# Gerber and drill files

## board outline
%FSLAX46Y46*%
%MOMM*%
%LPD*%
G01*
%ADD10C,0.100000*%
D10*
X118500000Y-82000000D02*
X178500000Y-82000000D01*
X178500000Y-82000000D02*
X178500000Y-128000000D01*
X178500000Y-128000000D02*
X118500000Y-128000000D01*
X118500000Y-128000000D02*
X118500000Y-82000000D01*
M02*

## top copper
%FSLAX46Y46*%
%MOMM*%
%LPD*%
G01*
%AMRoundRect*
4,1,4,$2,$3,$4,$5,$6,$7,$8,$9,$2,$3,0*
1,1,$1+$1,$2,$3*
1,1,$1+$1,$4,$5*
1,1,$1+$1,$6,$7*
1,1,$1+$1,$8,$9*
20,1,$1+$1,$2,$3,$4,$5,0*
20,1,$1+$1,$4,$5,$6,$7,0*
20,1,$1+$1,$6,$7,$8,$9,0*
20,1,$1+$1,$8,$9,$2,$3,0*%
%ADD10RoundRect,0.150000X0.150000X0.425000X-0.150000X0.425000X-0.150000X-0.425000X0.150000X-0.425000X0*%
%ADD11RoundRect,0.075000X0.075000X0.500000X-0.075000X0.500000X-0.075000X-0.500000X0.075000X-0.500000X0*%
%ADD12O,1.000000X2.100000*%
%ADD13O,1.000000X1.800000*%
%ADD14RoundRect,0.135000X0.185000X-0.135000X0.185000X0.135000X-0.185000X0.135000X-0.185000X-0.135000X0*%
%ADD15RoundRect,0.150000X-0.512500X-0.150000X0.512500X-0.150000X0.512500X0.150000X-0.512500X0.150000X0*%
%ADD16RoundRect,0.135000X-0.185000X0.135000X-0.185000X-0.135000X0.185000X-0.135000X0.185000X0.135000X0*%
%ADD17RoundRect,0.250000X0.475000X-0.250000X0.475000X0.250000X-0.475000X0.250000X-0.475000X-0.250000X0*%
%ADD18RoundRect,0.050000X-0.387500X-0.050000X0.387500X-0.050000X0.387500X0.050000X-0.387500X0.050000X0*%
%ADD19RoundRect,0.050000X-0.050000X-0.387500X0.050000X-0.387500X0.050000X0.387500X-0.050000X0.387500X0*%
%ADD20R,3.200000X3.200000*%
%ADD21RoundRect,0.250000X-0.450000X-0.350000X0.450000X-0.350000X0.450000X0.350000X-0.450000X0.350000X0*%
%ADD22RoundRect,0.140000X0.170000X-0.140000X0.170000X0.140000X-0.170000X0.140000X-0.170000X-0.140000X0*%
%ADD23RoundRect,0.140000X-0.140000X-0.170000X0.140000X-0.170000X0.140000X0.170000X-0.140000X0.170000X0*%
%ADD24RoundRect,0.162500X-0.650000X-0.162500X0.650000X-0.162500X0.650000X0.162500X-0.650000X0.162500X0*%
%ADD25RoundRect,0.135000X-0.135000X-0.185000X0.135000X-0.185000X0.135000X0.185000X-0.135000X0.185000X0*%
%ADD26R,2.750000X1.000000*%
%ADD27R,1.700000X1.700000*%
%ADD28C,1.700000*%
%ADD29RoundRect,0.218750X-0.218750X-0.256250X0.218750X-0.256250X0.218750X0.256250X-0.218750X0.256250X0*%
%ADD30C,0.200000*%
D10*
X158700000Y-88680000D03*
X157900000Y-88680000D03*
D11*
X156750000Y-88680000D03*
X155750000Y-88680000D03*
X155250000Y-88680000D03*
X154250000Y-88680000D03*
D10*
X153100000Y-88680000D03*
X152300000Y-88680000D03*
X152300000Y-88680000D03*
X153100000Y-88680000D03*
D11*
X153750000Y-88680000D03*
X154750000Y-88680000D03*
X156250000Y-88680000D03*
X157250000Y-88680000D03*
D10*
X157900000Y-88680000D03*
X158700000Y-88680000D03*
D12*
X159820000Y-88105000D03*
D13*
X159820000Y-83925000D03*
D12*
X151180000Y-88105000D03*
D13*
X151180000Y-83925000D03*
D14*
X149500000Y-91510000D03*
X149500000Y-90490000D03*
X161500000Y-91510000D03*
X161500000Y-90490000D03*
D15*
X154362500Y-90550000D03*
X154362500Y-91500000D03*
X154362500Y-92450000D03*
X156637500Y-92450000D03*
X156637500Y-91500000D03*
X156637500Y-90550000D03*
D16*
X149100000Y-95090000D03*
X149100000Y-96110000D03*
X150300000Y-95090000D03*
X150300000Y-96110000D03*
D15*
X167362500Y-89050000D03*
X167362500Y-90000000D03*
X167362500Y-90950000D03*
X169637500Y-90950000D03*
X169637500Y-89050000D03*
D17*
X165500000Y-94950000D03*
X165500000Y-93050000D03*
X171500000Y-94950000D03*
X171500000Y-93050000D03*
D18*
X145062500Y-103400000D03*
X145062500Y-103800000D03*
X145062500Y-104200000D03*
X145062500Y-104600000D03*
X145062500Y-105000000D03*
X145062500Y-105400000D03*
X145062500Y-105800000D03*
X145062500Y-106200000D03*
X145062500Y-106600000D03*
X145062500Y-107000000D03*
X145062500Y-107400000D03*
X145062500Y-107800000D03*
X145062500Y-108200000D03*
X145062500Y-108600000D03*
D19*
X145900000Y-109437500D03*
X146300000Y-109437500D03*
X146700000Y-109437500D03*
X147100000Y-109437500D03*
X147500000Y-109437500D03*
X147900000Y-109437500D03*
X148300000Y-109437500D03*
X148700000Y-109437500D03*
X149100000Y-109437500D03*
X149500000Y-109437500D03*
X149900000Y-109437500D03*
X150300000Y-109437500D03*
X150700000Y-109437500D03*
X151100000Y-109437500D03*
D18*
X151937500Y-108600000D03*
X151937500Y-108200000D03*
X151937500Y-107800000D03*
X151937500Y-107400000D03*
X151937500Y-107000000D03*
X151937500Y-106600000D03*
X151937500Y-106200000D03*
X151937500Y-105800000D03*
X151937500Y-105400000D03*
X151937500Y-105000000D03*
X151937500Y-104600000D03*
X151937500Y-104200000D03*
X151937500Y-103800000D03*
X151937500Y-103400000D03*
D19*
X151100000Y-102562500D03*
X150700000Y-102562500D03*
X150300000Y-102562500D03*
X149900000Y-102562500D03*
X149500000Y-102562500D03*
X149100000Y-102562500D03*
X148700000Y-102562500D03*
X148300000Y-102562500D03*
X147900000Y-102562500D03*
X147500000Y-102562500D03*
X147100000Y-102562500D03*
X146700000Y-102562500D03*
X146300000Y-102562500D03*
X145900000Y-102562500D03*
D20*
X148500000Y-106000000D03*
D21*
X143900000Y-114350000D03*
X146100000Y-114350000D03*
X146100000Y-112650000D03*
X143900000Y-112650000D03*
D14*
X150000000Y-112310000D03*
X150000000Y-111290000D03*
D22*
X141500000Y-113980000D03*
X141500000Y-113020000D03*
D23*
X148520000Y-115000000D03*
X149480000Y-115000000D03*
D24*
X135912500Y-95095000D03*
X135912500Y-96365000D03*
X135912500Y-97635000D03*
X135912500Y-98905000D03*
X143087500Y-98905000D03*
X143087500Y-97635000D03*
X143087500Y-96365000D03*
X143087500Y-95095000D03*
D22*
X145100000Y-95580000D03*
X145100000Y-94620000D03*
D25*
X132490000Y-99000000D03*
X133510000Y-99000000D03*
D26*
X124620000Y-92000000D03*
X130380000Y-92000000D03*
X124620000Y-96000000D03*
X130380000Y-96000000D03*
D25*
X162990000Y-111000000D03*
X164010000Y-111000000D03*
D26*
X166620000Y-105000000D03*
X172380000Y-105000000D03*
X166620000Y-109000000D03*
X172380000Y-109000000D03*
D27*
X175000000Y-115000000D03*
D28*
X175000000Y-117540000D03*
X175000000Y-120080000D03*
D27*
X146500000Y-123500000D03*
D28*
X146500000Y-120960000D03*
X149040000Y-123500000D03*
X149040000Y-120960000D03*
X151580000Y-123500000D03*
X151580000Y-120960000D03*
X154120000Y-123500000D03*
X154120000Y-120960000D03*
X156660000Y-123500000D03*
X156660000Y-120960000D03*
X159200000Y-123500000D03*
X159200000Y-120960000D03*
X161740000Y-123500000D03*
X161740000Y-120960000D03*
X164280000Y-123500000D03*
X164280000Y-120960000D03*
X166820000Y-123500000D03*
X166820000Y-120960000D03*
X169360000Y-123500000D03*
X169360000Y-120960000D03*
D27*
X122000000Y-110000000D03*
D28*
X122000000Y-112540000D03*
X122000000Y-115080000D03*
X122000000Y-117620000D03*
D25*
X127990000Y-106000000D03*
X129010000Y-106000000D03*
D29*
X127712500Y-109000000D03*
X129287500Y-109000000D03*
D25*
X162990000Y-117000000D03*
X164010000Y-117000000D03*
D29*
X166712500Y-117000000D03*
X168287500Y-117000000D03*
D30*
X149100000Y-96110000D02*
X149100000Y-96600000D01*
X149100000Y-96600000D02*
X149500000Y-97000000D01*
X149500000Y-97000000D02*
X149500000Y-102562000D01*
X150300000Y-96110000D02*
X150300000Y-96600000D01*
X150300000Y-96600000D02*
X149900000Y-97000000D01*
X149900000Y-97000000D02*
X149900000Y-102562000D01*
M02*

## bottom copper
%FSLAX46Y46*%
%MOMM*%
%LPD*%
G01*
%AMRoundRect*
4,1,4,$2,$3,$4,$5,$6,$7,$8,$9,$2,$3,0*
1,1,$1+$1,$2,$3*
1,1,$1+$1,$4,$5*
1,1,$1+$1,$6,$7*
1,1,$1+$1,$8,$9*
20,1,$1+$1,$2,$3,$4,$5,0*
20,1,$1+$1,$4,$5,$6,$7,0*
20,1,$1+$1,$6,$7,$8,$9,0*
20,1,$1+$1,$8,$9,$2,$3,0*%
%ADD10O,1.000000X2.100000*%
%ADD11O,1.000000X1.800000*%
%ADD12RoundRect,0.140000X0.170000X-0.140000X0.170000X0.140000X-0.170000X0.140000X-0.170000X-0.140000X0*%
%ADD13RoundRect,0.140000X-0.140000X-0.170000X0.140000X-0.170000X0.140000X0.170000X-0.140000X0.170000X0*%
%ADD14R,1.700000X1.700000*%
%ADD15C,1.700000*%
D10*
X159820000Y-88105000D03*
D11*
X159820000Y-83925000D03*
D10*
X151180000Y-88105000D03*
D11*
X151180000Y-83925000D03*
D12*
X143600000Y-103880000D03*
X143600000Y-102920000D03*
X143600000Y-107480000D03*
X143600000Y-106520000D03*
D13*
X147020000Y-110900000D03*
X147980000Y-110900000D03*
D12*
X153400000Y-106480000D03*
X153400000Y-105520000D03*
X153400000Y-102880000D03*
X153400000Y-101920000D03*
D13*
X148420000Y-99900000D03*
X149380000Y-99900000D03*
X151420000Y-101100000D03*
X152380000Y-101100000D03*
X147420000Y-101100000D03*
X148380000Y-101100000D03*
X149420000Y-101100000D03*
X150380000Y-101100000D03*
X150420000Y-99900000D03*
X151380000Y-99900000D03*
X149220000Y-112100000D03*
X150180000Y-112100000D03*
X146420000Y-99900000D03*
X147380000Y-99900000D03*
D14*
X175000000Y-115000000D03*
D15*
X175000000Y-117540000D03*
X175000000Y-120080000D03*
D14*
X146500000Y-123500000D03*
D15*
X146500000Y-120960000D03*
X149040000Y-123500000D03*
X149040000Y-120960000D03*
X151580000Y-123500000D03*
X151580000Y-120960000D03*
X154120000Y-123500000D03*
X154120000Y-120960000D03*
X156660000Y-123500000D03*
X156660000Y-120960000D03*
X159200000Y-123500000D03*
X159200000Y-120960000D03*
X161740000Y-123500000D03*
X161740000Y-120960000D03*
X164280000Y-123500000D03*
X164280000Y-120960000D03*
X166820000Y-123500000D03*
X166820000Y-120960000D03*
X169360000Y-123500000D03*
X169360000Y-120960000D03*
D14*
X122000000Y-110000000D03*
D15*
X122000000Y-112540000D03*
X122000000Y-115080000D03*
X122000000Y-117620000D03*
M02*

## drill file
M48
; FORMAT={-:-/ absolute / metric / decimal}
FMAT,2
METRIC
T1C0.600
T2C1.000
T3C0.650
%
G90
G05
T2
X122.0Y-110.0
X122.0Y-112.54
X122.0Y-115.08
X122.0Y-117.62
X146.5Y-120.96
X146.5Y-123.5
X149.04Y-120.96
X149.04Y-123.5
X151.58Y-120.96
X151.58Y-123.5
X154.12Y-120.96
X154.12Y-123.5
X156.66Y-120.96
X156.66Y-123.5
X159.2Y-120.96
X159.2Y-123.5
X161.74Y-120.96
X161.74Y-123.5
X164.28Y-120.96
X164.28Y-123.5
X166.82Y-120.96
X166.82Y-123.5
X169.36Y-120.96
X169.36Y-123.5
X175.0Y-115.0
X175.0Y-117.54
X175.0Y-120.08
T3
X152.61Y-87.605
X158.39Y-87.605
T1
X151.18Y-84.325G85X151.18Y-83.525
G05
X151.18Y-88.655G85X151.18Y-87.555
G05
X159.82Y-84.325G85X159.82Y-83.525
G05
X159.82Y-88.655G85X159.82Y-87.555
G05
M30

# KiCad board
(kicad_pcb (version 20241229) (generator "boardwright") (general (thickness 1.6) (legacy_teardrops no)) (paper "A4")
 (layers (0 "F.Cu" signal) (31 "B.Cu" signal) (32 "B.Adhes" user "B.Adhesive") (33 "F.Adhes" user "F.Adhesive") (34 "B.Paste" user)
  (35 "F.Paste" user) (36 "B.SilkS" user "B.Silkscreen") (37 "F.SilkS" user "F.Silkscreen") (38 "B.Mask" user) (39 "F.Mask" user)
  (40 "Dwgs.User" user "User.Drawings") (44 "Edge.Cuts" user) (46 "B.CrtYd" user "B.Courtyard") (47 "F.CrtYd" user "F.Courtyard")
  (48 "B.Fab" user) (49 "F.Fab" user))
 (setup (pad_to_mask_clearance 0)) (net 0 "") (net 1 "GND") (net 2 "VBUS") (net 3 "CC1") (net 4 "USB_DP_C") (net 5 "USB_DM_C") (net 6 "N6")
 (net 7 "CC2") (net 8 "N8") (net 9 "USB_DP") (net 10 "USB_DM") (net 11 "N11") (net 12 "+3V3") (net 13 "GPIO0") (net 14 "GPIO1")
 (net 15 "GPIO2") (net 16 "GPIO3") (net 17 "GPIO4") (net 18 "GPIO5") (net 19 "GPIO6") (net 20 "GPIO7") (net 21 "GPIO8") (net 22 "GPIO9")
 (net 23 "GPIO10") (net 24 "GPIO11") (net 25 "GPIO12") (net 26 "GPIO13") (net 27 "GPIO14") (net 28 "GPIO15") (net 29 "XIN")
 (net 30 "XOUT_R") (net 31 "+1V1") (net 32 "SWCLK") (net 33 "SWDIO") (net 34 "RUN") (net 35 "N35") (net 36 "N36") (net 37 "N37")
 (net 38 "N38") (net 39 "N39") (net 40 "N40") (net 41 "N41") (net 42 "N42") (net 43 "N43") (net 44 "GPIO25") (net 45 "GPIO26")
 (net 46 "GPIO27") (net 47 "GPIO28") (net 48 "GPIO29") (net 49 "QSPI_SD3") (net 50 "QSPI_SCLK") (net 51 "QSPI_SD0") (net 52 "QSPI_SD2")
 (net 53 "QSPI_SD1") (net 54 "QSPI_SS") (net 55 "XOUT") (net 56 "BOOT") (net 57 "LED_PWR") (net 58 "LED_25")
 (gr_line (start 118.5 82) (end 178.5 82) (stroke (width 0.1) (type default)) (layer "Edge.Cuts"))
 (gr_line (start 178.5 82) (end 178.5 128) (stroke (width 0.1) (type default)) (layer "Edge.Cuts"))
 (gr_line (start 178.5 128) (end 118.5 128) (stroke (width 0.1) (type default)) (layer "Edge.Cuts"))
 (gr_line (start 118.5 128) (end 118.5 82) (stroke (width 0.1) (type default)) (layer "Edge.Cuts"))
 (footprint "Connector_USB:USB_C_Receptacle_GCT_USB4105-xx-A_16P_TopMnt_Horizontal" (layer "F.Cu") (at 155.5 85 180)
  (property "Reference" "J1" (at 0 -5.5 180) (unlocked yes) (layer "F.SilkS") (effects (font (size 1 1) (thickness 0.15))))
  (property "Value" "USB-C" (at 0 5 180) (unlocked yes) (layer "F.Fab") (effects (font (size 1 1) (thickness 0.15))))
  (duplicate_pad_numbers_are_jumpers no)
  (pad "" np_thru_hole circle (at -2.89 -2.605 180) (size 0.65 0.65) (drill 0.65) (layers "*.Cu" "*.Mask"))
  (pad "" np_thru_hole circle (at 2.89 -2.605 180) (size 0.65 0.65) (drill 0.65) (layers "*.Cu" "*.Mask"))
  (pad "A1" smd roundrect (at -3.2 -3.68 180) (size 0.6 1.15) (layers "F.Cu" "F.Mask" "F.Paste") (roundrect_rratio 0.25) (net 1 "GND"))
  (pad "A4" smd roundrect (at -2.4 -3.68 180) (size 0.6 1.15) (layers "F.Cu" "F.Mask" "F.Paste") (roundrect_rratio 0.25) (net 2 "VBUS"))
  (pad "A5" smd roundrect (at -1.25 -3.68 180) (size 0.3 1.15) (layers "F.Cu" "F.Mask" "F.Paste") (roundrect_rratio 0.25) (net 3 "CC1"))
  (pad "A6" smd roundrect (at -0.25 -3.68 180) (size 0.3 1.15) (layers "F.Cu" "F.Mask" "F.Paste") (roundrect_rratio 0.25) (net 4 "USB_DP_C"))
  (pad "A7" smd roundrect (at 0.25 -3.68 180) (size 0.3 1.15) (layers "F.Cu" "F.Mask" "F.Paste") (roundrect_rratio 0.25) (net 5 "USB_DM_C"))
  (pad "A8" smd roundrect (at 1.25 -3.68 180) (size 0.3 1.15) (layers "F.Cu" "F.Mask" "F.Paste") (roundrect_rratio 0.25) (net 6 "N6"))
  (pad "A9" smd roundrect (at 2.4 -3.68 180) (size 0.6 1.15) (layers "F.Cu" "F.Mask" "F.Paste") (roundrect_rratio 0.25) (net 2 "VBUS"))
  (pad "A12" smd roundrect (at 3.2 -3.68 180) (size 0.6 1.15) (layers "F.Cu" "F.Mask" "F.Paste") (roundrect_rratio 0.25) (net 1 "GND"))
  (pad "B1" smd roundrect (at 3.2 -3.68 180) (size 0.6 1.15) (layers "F.Cu" "F.Mask" "F.Paste") (roundrect_rratio 0.25) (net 1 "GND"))
  (pad "B4" smd roundrect (at 2.4 -3.68 180) (size 0.6 1.15) (layers "F.Cu" "F.Mask" "F.Paste") (roundrect_rratio 0.25) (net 2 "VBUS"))
  (pad "B5" smd roundrect (at 1.75 -3.68 180) (size 0.3 1.15) (layers "F.Cu" "F.Mask" "F.Paste") (roundrect_rratio 0.25) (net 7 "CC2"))
  (pad "B6" smd roundrect (at 0.75 -3.68 180) (size 0.3 1.15) (layers "F.Cu" "F.Mask" "F.Paste") (roundrect_rratio 0.25) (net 4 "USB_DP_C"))
  (pad "B7" smd roundrect (at -0.75 -3.68 180) (size 0.3 1.15) (layers "F.Cu" "F.Mask" "F.Paste") (roundrect_rratio 0.25) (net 5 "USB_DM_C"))
  (pad "B8" smd roundrect (at -1.75 -3.68 180) (size 0.3 1.15) (layers "F.Cu" "F.Mask" "F.Paste") (roundrect_rratio 0.25) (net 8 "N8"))
  (pad "B9" smd roundrect (at -2.4 -3.68 180) (size 0.6 1.15) (layers "F.Cu" "F.Mask" "F.Paste") (roundrect_rratio 0.25) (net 2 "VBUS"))
  (pad "B12" smd roundrect (at -3.2 -3.68 180) (size 0.6 1.15) (layers "F.Cu" "F.Mask" "F.Paste") (roundrect_rratio 0.25) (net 1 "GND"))
  (pad "SH" thru_hole oval (at -4.32 -3.105 180) (size 1 2.1) (drill oval 0.6 1.7) (layers "*.Cu" "*.Mask" "F.Paste")
   (remove_unused_layers no) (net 1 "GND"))
  (pad "SH" thru_hole oval (at -4.32 1.075 180) (size 1 1.8) (drill oval 0.6 1.4) (layers "*.Cu" "*.Mask" "F.Paste")
   (remove_unused_layers no) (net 1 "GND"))
  (pad "SH" thru_hole oval (at 4.32 -3.105 180) (size 1 2.1) (drill oval 0.6 1.7) (layers "*.Cu" "*.Mask" "F.Paste")
   (remove_unused_layers no) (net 1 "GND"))
  (pad "SH" thru_hole oval (at 4.32 1.075 180) (size 1 1.8) (drill oval 0.6 1.4) (layers "*.Cu" "*.Mask" "F.Paste")
   (remove_unused_layers no) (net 1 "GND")))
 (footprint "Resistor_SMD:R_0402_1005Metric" (layer "F.Cu") (at 149.5 91 90)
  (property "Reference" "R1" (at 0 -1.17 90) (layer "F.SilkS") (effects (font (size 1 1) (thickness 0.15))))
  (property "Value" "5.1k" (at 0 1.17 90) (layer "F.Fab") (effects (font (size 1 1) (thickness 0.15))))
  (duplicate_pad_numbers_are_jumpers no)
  (pad "1" smd roundrect (at -0.51 0 90) (size 0.54 0.64) (layers "F.Cu" "F.Mask" "F.Paste") (roundrect_rratio 0.25) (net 3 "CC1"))
  (pad "2" smd roundrect (at 0.51 0 90) (size 0.54 0.64) (layers "F.Cu" "F.Mask" "F.Paste") (roundrect_rratio 0.25) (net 1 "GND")))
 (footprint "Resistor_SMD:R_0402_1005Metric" (layer "F.Cu") (at 161.5 91 90)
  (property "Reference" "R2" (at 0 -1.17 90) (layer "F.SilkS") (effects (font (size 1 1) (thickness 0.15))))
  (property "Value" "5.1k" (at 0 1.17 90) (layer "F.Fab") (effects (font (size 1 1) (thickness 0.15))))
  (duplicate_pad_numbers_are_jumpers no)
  (pad "1" smd roundrect (at -0.51 0 90) (size 0.54 0.64) (layers "F.Cu" "F.Mask" "F.Paste") (roundrect_rratio 0.25) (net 7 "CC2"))
  (pad "2" smd roundrect (at 0.51 0 90) (size 0.54 0.64) (layers "F.Cu" "F.Mask" "F.Paste") (roundrect_rratio 0.25) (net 1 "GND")))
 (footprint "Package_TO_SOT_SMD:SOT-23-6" (layer "F.Cu") (at 155.5 91.5)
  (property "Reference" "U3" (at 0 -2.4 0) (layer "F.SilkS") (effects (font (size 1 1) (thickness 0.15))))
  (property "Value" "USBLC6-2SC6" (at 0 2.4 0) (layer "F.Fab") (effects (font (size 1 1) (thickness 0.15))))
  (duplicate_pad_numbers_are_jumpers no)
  (pad "1" smd roundrect (at -1.1375 -0.95) (size 1.325 0.6) (layers "F.Cu" "F.Mask" "F.Paste") (roundrect_rratio 0.25) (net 4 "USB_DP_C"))
  (pad "2" smd roundrect (at -1.1375 0) (size 1.325 0.6) (layers "F.Cu" "F.Mask" "F.Paste") (roundrect_rratio 0.25) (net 1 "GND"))
  (pad "3" smd roundrect (at -1.1375 0.95) (size 1.325 0.6) (layers "F.Cu" "F.Mask" "F.Paste") (roundrect_rratio 0.25) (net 5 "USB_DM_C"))
  (pad "4" smd roundrect (at 1.1375 0.95) (size 1.325 0.6) (layers "F.Cu" "F.Mask" "F.Paste") (roundrect_rratio 0.25) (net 5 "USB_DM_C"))
  (pad "5" smd roundrect (at 1.1375 0) (size 1.325 0.6) (layers "F.Cu" "F.Mask" "F.Paste") (roundrect_rratio 0.25) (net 2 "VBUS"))
  (pad "6" smd roundrect (at 1.1375 -0.95) (size 1.325 0.6) (layers "F.Cu" "F.Mask" "F.Paste") (roundrect_rratio 0.25) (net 4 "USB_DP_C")))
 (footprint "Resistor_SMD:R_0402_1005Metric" (layer "F.Cu") (at 149.1 95.6 -90)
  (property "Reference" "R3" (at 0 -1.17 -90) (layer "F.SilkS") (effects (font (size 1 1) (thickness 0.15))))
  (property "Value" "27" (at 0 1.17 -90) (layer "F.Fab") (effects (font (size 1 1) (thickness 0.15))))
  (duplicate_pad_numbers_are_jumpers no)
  (pad "1" smd roundrect (at -0.51 0 -90) (size 0.54 0.64) (layers "F.Cu" "F.Mask" "F.Paste") (roundrect_rratio 0.25) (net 4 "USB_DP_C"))
  (pad "2" smd roundrect (at 0.51 0 -90) (size 0.54 0.64) (layers "F.Cu" "F.Mask" "F.Paste") (roundrect_rratio 0.25) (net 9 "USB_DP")))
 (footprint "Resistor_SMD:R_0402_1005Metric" (layer "F.Cu") (at 150.3 95.6 -90)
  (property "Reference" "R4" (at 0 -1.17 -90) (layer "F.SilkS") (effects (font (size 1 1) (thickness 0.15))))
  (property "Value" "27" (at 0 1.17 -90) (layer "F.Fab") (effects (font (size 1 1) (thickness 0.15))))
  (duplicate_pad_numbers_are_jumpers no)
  (pad "1" smd roundrect (at -0.51 0 -90) (size 0.54 0.64) (layers "F.Cu" "F.Mask" "F.Paste") (roundrect_rratio 0.25) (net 5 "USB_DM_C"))
  (pad "2" smd roundrect (at 0.51 0 -90) (size 0.54 0.64) (layers "F.Cu" "F.Mask" "F.Paste") (roundrect_rratio 0.25) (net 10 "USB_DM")))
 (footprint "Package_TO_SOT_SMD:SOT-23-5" (layer "F.Cu") (at 168.5 90)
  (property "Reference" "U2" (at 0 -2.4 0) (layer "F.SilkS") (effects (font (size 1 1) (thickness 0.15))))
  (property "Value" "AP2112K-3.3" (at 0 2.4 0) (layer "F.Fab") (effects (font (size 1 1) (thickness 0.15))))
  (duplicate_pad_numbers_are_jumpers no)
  (pad "1" smd roundrect (at -1.1375 -0.95) (size 1.325 0.6) (layers "F.Cu" "F.Mask" "F.Paste") (roundrect_rratio 0.25) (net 2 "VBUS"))
  (pad "2" smd roundrect (at -1.1375 0) (size 1.325 0.6) (layers "F.Cu" "F.Mask" "F.Paste") (roundrect_rratio 0.25) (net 1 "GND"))
  (pad "3" smd roundrect (at -1.1375 0.95) (size 1.325 0.6) (layers "F.Cu" "F.Mask" "F.Paste") (roundrect_rratio 0.25) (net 2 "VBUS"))
  (pad "4" smd roundrect (at 1.1375 0.95) (size 1.325 0.6) (layers "F.Cu" "F.Mask" "F.Paste") (roundrect_rratio 0.25) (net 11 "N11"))
  (pad "5" smd roundrect (at 1.1375 -0.95) (size 1.325 0.6) (layers "F.Cu" "F.Mask" "F.Paste") (roundrect_rratio 0.25) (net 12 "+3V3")))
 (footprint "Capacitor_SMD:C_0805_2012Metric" (layer "F.Cu") (at 165.5 94 90)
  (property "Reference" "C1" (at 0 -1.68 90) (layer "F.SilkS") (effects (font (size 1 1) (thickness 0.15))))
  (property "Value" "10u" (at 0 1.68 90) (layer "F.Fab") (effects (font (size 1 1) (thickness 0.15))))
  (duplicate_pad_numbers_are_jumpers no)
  (pad "1" smd roundrect (at -0.95 0 90) (size 1 1.45) (layers "F.Cu" "F.Mask" "F.Paste") (roundrect_rratio 0.25) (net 2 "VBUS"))
  (pad "2" smd roundrect (at 0.95 0 90) (size 1 1.45) (layers "F.Cu" "F.Mask" "F.Paste") (roundrect_rratio 0.25) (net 1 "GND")))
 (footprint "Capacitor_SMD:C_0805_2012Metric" (layer "F.Cu") (at 171.5 94 90)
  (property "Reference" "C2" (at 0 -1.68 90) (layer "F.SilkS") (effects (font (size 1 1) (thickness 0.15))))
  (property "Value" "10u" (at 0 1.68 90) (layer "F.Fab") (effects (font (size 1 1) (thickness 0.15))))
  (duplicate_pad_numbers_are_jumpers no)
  (pad "1" smd roundrect (at -0.95 0 90) (size 1 1.45) (layers "F.Cu" "F.Mask" "F.Paste") (roundrect_rratio 0.25) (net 12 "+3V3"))
  (pad "2" smd roundrect (at 0.95 0 90) (size 1 1.45) (layers "F.Cu" "F.Mask" "F.Paste") (roundrect_rratio 0.25) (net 1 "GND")))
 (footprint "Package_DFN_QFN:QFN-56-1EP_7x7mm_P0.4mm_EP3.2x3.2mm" (layer "F.Cu") (at 148.5 106)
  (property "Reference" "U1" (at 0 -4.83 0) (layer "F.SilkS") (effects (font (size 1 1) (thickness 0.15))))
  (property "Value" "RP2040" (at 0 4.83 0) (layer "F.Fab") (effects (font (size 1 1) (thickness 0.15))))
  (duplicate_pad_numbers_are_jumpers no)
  (pad "" smd roundrect (at -0.8 -0.8) (size 1.29 1.29) (layers "F.Paste") (roundrect_rratio 0.193798))
  (pad "" smd roundrect (at -0.8 0.8) (size 1.29 1.29) (layers "F.Paste") (roundrect_rratio 0.193798))
  (pad "" smd roundrect (at 0.8 -0.8) (size 1.29 1.29) (layers "F.Paste") (roundrect_rratio 0.193798))
  (pad "" smd roundrect (at 0.8 0.8) (size 1.29 1.29) (layers "F.Paste") (roundrect_rratio 0.193798))
  (pad "1" smd roundrect (at -3.4375 -2.6) (size 0.875 0.2) (layers "F.Cu" "F.Mask" "F.Paste") (roundrect_rratio 0.25) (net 12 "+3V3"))
  (pad "2" smd roundrect (at -3.4375 -2.2) (size 0.875 0.2) (layers "F.Cu" "F.Mask" "F.Paste") (roundrect_rratio 0.25) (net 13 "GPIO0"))
  (pad "3" smd roundrect (at -3.4375 -1.8) (size 0.875 0.2) (layers "F.Cu" "F.Mask" "F.Paste") (roundrect_rratio 0.25) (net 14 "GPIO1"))
  (pad "4" smd roundrect (at -3.4375 -1.4) (size 0.875 0.2) (layers "F.Cu" "F.Mask" "F.Paste") (roundrect_rratio 0.25) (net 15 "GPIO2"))
  (pad "5" smd roundrect (at -3.4375 -1) (size 0.875 0.2) (layers "F.Cu" "F.Mask" "F.Paste") (roundrect_rratio 0.25) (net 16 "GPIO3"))
  (pad "6" smd roundrect (at -3.4375 -0.6) (size 0.875 0.2) (layers "F.Cu" "F.Mask" "F.Paste") (roundrect_rratio 0.25) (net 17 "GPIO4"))
  (pad "7" smd roundrect (at -3.4375 -0.2) (size 0.875 0.2) (layers "F.Cu" "F.Mask" "F.Paste") (roundrect_rratio 0.25) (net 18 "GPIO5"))
  (pad "8" smd roundrect (at -3.4375 0.2) (size 0.875 0.2) (layers "F.Cu" "F.Mask" "F.Paste") (roundrect_rratio 0.25) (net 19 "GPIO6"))
  (pad "9" smd roundrect (at -3.4375 0.6) (size 0.875 0.2) (layers "F.Cu" "F.Mask" "F.Paste") (roundrect_rratio 0.25) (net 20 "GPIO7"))
  (pad "10" smd roundrect (at -3.4375 1) (size 0.875 0.2) (layers "F.Cu" "F.Mask" "F.Paste") (roundrect_rratio 0.25) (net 12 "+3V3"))
  (pad "11" smd roundrect (at -3.4375 1.4) (size 0.875 0.2) (layers "F.Cu" "F.Mask" "F.Paste") (roundrect_rratio 0.25) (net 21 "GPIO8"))
  (pad "12" smd roundrect (at -3.4375 1.8) (size 0.875 0.2) (layers "F.Cu" "F.Mask" "F.Paste") (roundrect_rratio 0.25) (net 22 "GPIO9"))
  (pad "13" smd roundrect (at -3.4375 2.2) (size 0.875 0.2) (layers "F.Cu" "F.Mask" "F.Paste") (roundrect_rratio 0.25) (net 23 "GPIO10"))
  (pad "14" smd roundrect (at -3.4375 2.6) (size 0.875 0.2) (layers "F.Cu" "F.Mask" "F.Paste") (roundrect_rratio 0.25) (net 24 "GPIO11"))
  (pad "15" smd roundrect (at -2.6 3.4375) (size 0.2 0.875) (layers "F.Cu" "F.Mask" "F.Paste") (roundrect_rratio 0.25) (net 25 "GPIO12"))
  (pad "16" smd roundrect (at -2.2 3.4375) (size 0.2 0.875) (layers "F.Cu" "F.Mask" "F.Paste") (roundrect_rratio 0.25) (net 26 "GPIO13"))
  (pad "17" smd roundrect (at -1.8 3.4375) (size 0.2 0.875) (layers "F.Cu" "F.Mask" "F.Paste") (roundrect_rratio 0.25) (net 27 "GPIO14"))
  (pad "18" smd roundrect (at -1.4 3.4375) (size 0.2 0.875) (layers "F.Cu" "F.Mask" "F.Paste") (roundrect_rratio 0.25) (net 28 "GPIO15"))
  (pad "19" smd roundrect (at -1 3.4375) (size 0.2 0.875) (layers "F.Cu" "F.Mask" "F.Paste") (roundrect_rratio 0.25) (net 1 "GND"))
  (pad "20" smd roundrect (at -0.6 3.4375) (size 0.2 0.875) (layers "F.Cu" "F.Mask" "F.Paste") (roundrect_rratio 0.25) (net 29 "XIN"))
  (pad "21" smd roundrect (at -0.2 3.4375) (size 0.2 0.875) (layers "F.Cu" "F.Mask" "F.Paste") (roundrect_rratio 0.25) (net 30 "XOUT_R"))
  (pad "22" smd roundrect (at 0.2 3.4375) (size 0.2 0.875) (layers "F.Cu" "F.Mask" "F.Paste") (roundrect_rratio 0.25) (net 12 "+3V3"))
  (pad "23" smd roundrect (at 0.6 3.4375) (size 0.2 0.875) (layers "F.Cu" "F.Mask" "F.Paste") (roundrect_rratio 0.25) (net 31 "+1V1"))
  (pad "24" smd roundrect (at 1 3.4375) (size 0.2 0.875) (layers "F.Cu" "F.Mask" "F.Paste") (roundrect_rratio 0.25) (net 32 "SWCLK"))
  (pad "25" smd roundrect (at 1.4 3.4375) (size 0.2 0.875) (layers "F.Cu" "F.Mask" "F.Paste") (roundrect_rratio 0.25) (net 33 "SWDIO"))
  (pad "26" smd roundrect (at 1.8 3.4375) (size 0.2 0.875) (layers "F.Cu" "F.Mask" "F.Paste") (roundrect_rratio 0.25) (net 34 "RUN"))
  (pad "27" smd roundrect (at 2.2 3.4375) (size 0.2 0.875) (layers "F.Cu" "F.Mask" "F.Paste") (roundrect_rratio 0.25) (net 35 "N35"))
  (pad "28" smd roundrect (at 2.6 3.4375) (size 0.2 0.875) (layers "F.Cu" "F.Mask" "F.Paste") (roundrect_rratio 0.25) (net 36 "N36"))
  (pad "29" smd roundrect (at 3.4375 2.6) (size 0.875 0.2) (layers "F.Cu" "F.Mask" "F.Paste") (roundrect_rratio 0.25) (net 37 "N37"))
  (pad "30" smd roundrect (at 3.4375 2.2) (size 0.875 0.2) (layers "F.Cu" "F.Mask" "F.Paste") (roundrect_rratio 0.25) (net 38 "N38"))
  (pad "31" smd roundrect (at 3.4375 1.8) (size 0.875 0.2) (layers "F.Cu" "F.Mask" "F.Paste") (roundrect_rratio 0.25) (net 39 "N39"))
  (pad "32" smd roundrect (at 3.4375 1.4) (size 0.875 0.2) (layers "F.Cu" "F.Mask" "F.Paste") (roundrect_rratio 0.25) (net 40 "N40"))
  (pad "33" smd roundrect (at 3.4375 1) (size 0.875 0.2) (layers "F.Cu" "F.Mask" "F.Paste") (roundrect_rratio 0.25) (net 12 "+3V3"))
  (pad "34" smd roundrect (at 3.4375 0.6) (size 0.875 0.2) (layers "F.Cu" "F.Mask" "F.Paste") (roundrect_rratio 0.25) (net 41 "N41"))
  (pad "35" smd roundrect (at 3.4375 0.2) (size 0.875 0.2) (layers "F.Cu" "F.Mask" "F.Paste") (roundrect_rratio 0.25) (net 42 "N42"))
  (pad "36" smd roundrect (at 3.4375 -0.2) (size 0.875 0.2) (layers "F.Cu" "F.Mask" "F.Paste") (roundrect_rratio 0.25) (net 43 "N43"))
  (pad "37" smd roundrect (at 3.4375 -0.6) (size 0.875 0.2) (layers "F.Cu" "F.Mask" "F.Paste") (roundrect_rratio 0.25) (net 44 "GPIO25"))
  (pad "38" smd roundrect (at 3.4375 -1) (size 0.875 0.2) (layers "F.Cu" "F.Mask" "F.Paste") (roundrect_rratio 0.25) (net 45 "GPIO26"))
  (pad "39" smd roundrect (at 3.4375 -1.4) (size 0.875 0.2) (layers "F.Cu" "F.Mask" "F.Paste") (roundrect_rratio 0.25) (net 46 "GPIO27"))
  (pad "40" smd roundrect (at 3.4375 -1.8) (size 0.875 0.2) (layers "F.Cu" "F.Mask" "F.Paste") (roundrect_rratio 0.25) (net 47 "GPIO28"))
  (pad "41" smd roundrect (at 3.4375 -2.2) (size 0.875 0.2) (layers "F.Cu" "F.Mask" "F.Paste") (roundrect_rratio 0.25) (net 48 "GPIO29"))
  (pad "42" smd roundrect (at 3.4375 -2.6) (size 0.875 0.2) (layers "F.Cu" "F.Mask" "F.Paste") (roundrect_rratio 0.25) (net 12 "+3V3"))
  (pad "43" smd roundrect (at 2.6 -3.4375) (size 0.2 0.875) (layers "F.Cu" "F.Mask" "F.Paste") (roundrect_rratio 0.25) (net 12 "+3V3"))
  (pad "44" smd roundrect (at 2.2 -3.4375) (size 0.2 0.875) (layers "F.Cu" "F.Mask" "F.Paste") (roundrect_rratio 0.25) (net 12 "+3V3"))
  (pad "45" smd roundrect (at 1.8 -3.4375) (size 0.2 0.875) (layers "F.Cu" "F.Mask" "F.Paste") (roundrect_rratio 0.25) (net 31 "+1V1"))
  (pad "46" smd roundrect (at 1.4 -3.4375) (size 0.2 0.875) (layers "F.Cu" "F.Mask" "F.Paste") (roundrect_rratio 0.25) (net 10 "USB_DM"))
  (pad "47" smd roundrect (at 1 -3.4375) (size 0.2 0.875) (layers "F.Cu" "F.Mask" "F.Paste") (roundrect_rratio 0.25) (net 9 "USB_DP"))
  (pad "48" smd roundrect (at 0.6 -3.4375) (size 0.2 0.875) (layers "F.Cu" "F.Mask" "F.Paste") (roundrect_rratio 0.25) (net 12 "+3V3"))
  (pad "49" smd roundrect (at 0.2 -3.4375) (size 0.2 0.875) (layers "F.Cu" "F.Mask" "F.Paste") (roundrect_rratio 0.25) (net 12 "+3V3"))
  (pad "50" smd roundrect (at -0.2 -3.4375) (size 0.2 0.875) (layers "F.Cu" "F.Mask" "F.Paste") (roundrect_rratio 0.25) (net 31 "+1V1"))
  (pad "51" smd roundrect (at -0.6 -3.4375) (size 0.2 0.875) (layers "F.Cu" "F.Mask" "F.Paste") (roundrect_rratio 0.25) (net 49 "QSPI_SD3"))
  (pad "52" smd roundrect (at -1 -3.4375) (size 0.2 0.875) (layers "F.Cu" "F.Mask" "F.Paste") (roundrect_rratio 0.25) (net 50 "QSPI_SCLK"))
  (pad "53" smd roundrect (at -1.4 -3.4375) (size 0.2 0.875) (layers "F.Cu" "F.Mask" "F.Paste") (roundrect_rratio 0.25) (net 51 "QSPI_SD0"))
  (pad "54" smd roundrect (at -1.8 -3.4375) (size 0.2 0.875) (layers "F.Cu" "F.Mask" "F.Paste") (roundrect_rratio 0.25) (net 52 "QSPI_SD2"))
  (pad "55" smd roundrect (at -2.2 -3.4375) (size 0.2 0.875) (layers "F.Cu" "F.Mask" "F.Paste") (roundrect_rratio 0.25) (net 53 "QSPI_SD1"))
  (pad "56" smd roundrect (at -2.6 -3.4375) (size 0.2 0.875) (layers "F.Cu" "F.Mask" "F.Paste") (roundrect_rratio 0.25) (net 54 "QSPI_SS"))
  (pad "57" smd rect (at 0 0) (size 3.2 3.2) (layers "F.Cu" "F.Mask") (zone_connect 2) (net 1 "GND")))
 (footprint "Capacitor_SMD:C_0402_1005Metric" (layer "B.Cu") (at 143.6 103.4 90)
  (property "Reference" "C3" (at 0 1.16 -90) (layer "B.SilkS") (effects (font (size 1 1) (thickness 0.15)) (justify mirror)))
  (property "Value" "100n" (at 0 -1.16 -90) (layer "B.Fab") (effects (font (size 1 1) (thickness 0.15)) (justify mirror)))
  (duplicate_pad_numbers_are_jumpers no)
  (pad "1" smd roundrect (at -0.48 0 90) (size 0.56 0.62) (layers "B.Cu" "B.Mask" "B.Paste") (roundrect_rratio 0.25) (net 12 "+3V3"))
  (pad "2" smd roundrect (at 0.48 0 90) (size 0.56 0.62) (layers "B.Cu" "B.Mask" "B.Paste") (roundrect_rratio 0.25) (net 1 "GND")))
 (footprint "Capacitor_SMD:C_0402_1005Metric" (layer "B.Cu") (at 143.6 107 90)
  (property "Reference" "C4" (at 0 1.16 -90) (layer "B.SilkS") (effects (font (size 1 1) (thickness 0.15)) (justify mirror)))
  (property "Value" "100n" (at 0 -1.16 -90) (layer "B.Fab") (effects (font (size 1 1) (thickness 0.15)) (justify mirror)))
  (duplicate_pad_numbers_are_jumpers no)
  (pad "1" smd roundrect (at -0.48 0 90) (size 0.56 0.62) (layers "B.Cu" "B.Mask" "B.Paste") (roundrect_rratio 0.25) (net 12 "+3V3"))
  (pad "2" smd roundrect (at 0.48 0 90) (size 0.56 0.62) (layers "B.Cu" "B.Mask" "B.Paste") (roundrect_rratio 0.25) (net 1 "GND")))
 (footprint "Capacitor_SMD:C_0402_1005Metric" (layer "B.Cu") (at 147.5 110.9)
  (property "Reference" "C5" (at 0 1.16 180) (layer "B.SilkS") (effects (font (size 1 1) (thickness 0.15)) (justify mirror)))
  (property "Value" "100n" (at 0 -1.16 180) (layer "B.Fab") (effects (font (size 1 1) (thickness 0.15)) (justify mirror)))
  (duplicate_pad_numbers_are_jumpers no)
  (pad "1" smd roundrect (at -0.48 0) (size 0.56 0.62) (layers "B.Cu" "B.Mask" "B.Paste") (roundrect_rratio 0.25) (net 12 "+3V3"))
  (pad "2" smd roundrect (at 0.48 0) (size 0.56 0.62) (layers "B.Cu" "B.Mask" "B.Paste") (roundrect_rratio 0.25) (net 1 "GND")))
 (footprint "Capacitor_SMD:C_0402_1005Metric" (layer "B.Cu") (at 153.4 106 90)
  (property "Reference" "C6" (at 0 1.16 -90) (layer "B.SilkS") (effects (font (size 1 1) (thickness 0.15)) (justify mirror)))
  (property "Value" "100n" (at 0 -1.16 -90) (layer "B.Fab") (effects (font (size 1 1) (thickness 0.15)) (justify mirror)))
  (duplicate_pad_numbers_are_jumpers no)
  (pad "1" smd roundrect (at -0.48 0 90) (size 0.56 0.62) (layers "B.Cu" "B.Mask" "B.Paste") (roundrect_rratio 0.25) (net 12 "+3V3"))
  (pad "2" smd roundrect (at 0.48 0 90) (size 0.56 0.62) (layers "B.Cu" "B.Mask" "B.Paste") (roundrect_rratio 0.25) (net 1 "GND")))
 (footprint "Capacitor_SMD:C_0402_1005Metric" (layer "B.Cu") (at 153.4 102.4 90)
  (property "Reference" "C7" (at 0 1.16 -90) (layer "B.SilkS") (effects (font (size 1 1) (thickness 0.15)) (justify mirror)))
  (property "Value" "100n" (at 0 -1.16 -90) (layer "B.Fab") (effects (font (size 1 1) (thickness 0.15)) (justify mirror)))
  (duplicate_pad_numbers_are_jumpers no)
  (pad "1" smd roundrect (at -0.48 0 90) (size 0.56 0.62) (layers "B.Cu" "B.Mask" "B.Paste") (roundrect_rratio 0.25) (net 12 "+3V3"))
  (pad "2" smd roundrect (at 0.48 0 90) (size 0.56 0.62) (layers "B.Cu" "B.Mask" "B.Paste") (roundrect_rratio 0.25) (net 1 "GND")))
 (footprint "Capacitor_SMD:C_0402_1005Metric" (layer "B.Cu") (at 148.9 99.9)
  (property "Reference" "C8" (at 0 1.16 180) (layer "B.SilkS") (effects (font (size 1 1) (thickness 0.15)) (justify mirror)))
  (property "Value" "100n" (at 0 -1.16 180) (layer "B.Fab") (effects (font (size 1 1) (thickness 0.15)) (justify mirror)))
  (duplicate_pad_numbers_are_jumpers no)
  (pad "1" smd roundrect (at -0.48 0) (size 0.56 0.62) (layers "B.Cu" "B.Mask" "B.Paste") (roundrect_rratio 0.25) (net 12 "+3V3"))
  (pad "2" smd roundrect (at 0.48 0) (size 0.56 0.62) (layers "B.Cu" "B.Mask" "B.Paste") (roundrect_rratio 0.25) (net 1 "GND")))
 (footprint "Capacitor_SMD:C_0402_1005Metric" (layer "B.Cu") (at 151.9 101.1)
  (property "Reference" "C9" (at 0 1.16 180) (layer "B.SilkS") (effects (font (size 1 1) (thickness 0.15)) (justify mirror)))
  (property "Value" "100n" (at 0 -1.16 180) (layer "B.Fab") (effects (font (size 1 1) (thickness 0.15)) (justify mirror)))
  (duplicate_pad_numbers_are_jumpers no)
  (pad "1" smd roundrect (at -0.48 0) (size 0.56 0.62) (layers "B.Cu" "B.Mask" "B.Paste") (roundrect_rratio 0.25) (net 12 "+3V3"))
  (pad "2" smd roundrect (at 0.48 0) (size 0.56 0.62) (layers "B.Cu" "B.Mask" "B.Paste") (roundrect_rratio 0.25) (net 1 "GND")))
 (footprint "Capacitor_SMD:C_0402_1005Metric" (layer "B.Cu") (at 147.9 101.1)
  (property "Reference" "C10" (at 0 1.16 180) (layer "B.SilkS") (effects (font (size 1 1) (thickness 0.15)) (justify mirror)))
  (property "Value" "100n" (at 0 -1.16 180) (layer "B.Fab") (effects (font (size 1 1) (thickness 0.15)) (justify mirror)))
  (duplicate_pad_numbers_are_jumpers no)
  (pad "1" smd roundrect (at -0.48 0) (size 0.56 0.62) (layers "B.Cu" "B.Mask" "B.Paste") (roundrect_rratio 0.25) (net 12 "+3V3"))
  (pad "2" smd roundrect (at 0.48 0) (size 0.56 0.62) (layers "B.Cu" "B.Mask" "B.Paste") (roundrect_rratio 0.25) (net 1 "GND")))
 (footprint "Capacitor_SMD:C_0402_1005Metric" (layer "B.Cu") (at 149.9 101.1)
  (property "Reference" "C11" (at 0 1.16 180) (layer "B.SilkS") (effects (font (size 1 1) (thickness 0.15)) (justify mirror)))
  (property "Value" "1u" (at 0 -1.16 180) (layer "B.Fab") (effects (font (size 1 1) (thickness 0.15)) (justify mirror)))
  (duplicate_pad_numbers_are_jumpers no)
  (pad "1" smd roundrect (at -0.48 0) (size 0.56 0.62) (layers "B.Cu" "B.Mask" "B.Paste") (roundrect_rratio 0.25) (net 12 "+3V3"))
  (pad "2" smd roundrect (at 0.48 0) (size 0.56 0.62) (layers "B.Cu" "B.Mask" "B.Paste") (roundrect_rratio 0.25) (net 1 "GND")))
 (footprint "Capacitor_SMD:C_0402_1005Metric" (layer "B.Cu") (at 150.9 99.9)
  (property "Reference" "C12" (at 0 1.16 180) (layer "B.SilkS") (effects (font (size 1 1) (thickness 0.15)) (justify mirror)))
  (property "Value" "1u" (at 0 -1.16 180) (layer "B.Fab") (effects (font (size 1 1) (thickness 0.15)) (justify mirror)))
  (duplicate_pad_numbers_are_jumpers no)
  (pad "1" smd roundrect (at -0.48 0) (size 0.56 0.62) (layers "B.Cu" "B.Mask" "B.Paste") (roundrect_rratio 0.25) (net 31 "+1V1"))
  (pad "2" smd roundrect (at 0.48 0) (size 0.56 0.62) (layers "B.Cu" "B.Mask" "B.Paste") (roundrect_rratio 0.25) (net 1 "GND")))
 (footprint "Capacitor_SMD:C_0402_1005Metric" (layer "B.Cu") (at 149.7 112.1)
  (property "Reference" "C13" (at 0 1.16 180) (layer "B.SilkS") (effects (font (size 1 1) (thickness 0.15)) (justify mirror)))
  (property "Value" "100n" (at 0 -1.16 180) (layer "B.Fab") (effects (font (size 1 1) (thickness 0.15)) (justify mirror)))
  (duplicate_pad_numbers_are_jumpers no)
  (pad "1" smd roundrect (at -0.48 0) (size 0.56 0.62) (layers "B.Cu" "B.Mask" "B.Paste") (roundrect_rratio 0.25) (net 31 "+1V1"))
  (pad "2" smd roundrect (at 0.48 0) (size 0.56 0.62) (layers "B.Cu" "B.Mask" "B.Paste") (roundrect_rratio 0.25) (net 1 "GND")))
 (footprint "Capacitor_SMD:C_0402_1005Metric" (layer "B.Cu") (at 146.9 99.9)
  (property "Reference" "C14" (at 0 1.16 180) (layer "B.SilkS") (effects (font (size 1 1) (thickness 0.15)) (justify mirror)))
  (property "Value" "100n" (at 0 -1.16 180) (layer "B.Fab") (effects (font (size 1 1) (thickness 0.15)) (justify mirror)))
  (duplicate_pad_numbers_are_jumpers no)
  (pad "1" smd roundrect (at -0.48 0) (size 0.56 0.62) (layers "B.Cu" "B.Mask" "B.Paste") (roundrect_rratio 0.25) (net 31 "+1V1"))
  (pad "2" smd roundrect (at 0.48 0) (size 0.56 0.62) (layers "B.Cu" "B.Mask" "B.Paste") (roundrect_rratio 0.25) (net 1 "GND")))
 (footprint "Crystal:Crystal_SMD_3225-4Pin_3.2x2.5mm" (layer "F.Cu") (at 145 113.5)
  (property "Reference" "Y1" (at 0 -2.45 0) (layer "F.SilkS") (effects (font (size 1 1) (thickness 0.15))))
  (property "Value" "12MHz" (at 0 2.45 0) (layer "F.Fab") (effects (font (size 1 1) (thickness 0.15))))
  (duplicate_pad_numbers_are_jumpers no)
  (pad "1" smd roundrect (at -1.1 0.85) (size 1.4 1.2) (layers "F.Cu" "F.Mask" "F.Paste") (roundrect_rratio 0.208333) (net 29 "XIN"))
  (pad "2" smd roundrect (at 1.1 0.85) (size 1.4 1.2) (layers "F.Cu" "F.Mask" "F.Paste") (roundrect_rratio 0.208333) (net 1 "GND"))
  (pad "3" smd roundrect (at 1.1 -0.85) (size 1.4 1.2) (layers "F.Cu" "F.Mask" "F.Paste") (roundrect_rratio 0.208333) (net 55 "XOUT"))
  (pad "4" smd roundrect (at -1.1 -0.85) (size 1.4 1.2) (layers "F.Cu" "F.Mask" "F.Paste") (roundrect_rratio 0.208333) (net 1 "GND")))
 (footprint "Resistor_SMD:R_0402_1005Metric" (layer "F.Cu") (at 150 111.8 90)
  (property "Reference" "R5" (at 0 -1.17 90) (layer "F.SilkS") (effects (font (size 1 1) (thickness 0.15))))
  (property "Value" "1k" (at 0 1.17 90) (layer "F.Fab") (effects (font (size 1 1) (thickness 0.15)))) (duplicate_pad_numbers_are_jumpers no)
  (pad "1" smd roundrect (at -0.51 0 90) (size 0.54 0.64) (layers "F.Cu" "F.Mask" "F.Paste") (roundrect_rratio 0.25) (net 30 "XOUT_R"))
  (pad "2" smd roundrect (at 0.51 0 90) (size 0.54 0.64) (layers "F.Cu" "F.Mask" "F.Paste") (roundrect_rratio 0.25) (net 55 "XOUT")))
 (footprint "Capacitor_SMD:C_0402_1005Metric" (layer "F.Cu") (at 141.5 113.5 90)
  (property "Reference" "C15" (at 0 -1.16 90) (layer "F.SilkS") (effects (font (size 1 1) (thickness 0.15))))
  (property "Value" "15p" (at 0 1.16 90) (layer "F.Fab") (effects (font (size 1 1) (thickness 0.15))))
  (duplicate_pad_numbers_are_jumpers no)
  (pad "1" smd roundrect (at -0.48 0 90) (size 0.56 0.62) (layers "F.Cu" "F.Mask" "F.Paste") (roundrect_rratio 0.25) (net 29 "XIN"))
  (pad "2" smd roundrect (at 0.48 0 90) (size 0.56 0.62) (layers "F.Cu" "F.Mask" "F.Paste") (roundrect_rratio 0.25) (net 1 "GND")))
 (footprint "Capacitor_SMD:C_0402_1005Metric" (layer "F.Cu") (at 149 115)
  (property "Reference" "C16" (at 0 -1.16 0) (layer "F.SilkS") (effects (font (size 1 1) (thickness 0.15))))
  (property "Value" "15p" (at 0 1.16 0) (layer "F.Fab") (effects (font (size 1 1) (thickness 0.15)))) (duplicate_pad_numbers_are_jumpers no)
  (pad "1" smd roundrect (at -0.48 0) (size 0.56 0.62) (layers "F.Cu" "F.Mask" "F.Paste") (roundrect_rratio 0.25) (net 55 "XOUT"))
  (pad "2" smd roundrect (at 0.48 0) (size 0.56 0.62) (layers "F.Cu" "F.Mask" "F.Paste") (roundrect_rratio 0.25) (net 1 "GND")))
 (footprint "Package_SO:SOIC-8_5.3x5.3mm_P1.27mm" (layer "F.Cu") (at 139.5 97)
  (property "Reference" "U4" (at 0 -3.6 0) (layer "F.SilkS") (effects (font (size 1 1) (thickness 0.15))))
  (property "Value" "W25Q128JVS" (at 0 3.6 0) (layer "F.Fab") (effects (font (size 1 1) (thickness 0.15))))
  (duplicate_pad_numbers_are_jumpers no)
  (pad "1" smd roundrect (at -3.5875 -1.905) (size 1.625 0.65) (layers "F.Cu" "F.Mask" "F.Paste") (roundrect_rratio 0.25) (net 54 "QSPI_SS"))
  (pad "2" smd roundrect (at -3.5875 -0.635) (size 1.625 0.65) (layers "F.Cu" "F.Mask" "F.Paste") (roundrect_rratio 0.25)
   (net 53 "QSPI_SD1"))
  (pad "3" smd roundrect (at -3.5875 0.635) (size 1.625 0.65) (layers "F.Cu" "F.Mask" "F.Paste") (roundrect_rratio 0.25) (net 52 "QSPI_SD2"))
  (pad "4" smd roundrect (at -3.5875 1.905) (size 1.625 0.65) (layers "F.Cu" "F.Mask" "F.Paste") (roundrect_rratio 0.25) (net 1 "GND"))
  (pad "5" smd roundrect (at 3.5875 1.905) (size 1.625 0.65) (layers "F.Cu" "F.Mask" "F.Paste") (roundrect_rratio 0.25) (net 51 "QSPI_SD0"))
  (pad "6" smd roundrect (at 3.5875 0.635) (size 1.625 0.65) (layers "F.Cu" "F.Mask" "F.Paste") (roundrect_rratio 0.25) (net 50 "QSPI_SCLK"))
  (pad "7" smd roundrect (at 3.5875 -0.635) (size 1.625 0.65) (layers "F.Cu" "F.Mask" "F.Paste") (roundrect_rratio 0.25) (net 49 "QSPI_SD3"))
  (pad "8" smd roundrect (at 3.5875 -1.905) (size 1.625 0.65) (layers "F.Cu" "F.Mask" "F.Paste") (roundrect_rratio 0.25) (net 12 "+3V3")))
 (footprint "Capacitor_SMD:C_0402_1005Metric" (layer "F.Cu") (at 145.1 95.1 90)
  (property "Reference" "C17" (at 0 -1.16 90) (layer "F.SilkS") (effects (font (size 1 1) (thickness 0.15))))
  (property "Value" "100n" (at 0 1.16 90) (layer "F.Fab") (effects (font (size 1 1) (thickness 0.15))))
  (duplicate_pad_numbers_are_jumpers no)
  (pad "1" smd roundrect (at -0.48 0 90) (size 0.56 0.62) (layers "F.Cu" "F.Mask" "F.Paste") (roundrect_rratio 0.25) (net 12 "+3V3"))
  (pad "2" smd roundrect (at 0.48 0 90) (size 0.56 0.62) (layers "F.Cu" "F.Mask" "F.Paste") (roundrect_rratio 0.25) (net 1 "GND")))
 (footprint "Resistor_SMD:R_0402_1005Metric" (layer "F.Cu") (at 133 99)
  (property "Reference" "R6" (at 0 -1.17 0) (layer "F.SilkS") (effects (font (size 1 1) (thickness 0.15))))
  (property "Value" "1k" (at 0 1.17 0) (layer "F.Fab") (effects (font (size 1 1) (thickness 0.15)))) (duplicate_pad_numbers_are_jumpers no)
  (pad "1" smd roundrect (at -0.51 0) (size 0.54 0.64) (layers "F.Cu" "F.Mask" "F.Paste") (roundrect_rratio 0.25) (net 54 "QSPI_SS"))
  (pad "2" smd roundrect (at 0.51 0) (size 0.54 0.64) (layers "F.Cu" "F.Mask" "F.Paste") (roundrect_rratio 0.25) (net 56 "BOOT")))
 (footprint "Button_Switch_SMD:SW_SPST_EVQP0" (layer "F.Cu") (at 127.5 94)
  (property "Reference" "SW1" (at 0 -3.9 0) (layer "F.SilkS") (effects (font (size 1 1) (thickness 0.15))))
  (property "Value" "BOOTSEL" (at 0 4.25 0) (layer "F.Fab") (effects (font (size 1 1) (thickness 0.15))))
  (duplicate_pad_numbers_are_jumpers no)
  (pad "1" smd rect (at -2.88 -2) (size 2.75 1) (layers "F.Cu" "F.Mask" "F.Paste") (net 56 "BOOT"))
  (pad "1" smd rect (at 2.88 -2) (size 2.75 1) (layers "F.Cu" "F.Mask" "F.Paste") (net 56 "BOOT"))
  (pad "2" smd rect (at -2.88 2) (size 2.75 1) (layers "F.Cu" "F.Mask" "F.Paste") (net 1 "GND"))
  (pad "2" smd rect (at 2.88 2) (size 2.75 1) (layers "F.Cu" "F.Mask" "F.Paste") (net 1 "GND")))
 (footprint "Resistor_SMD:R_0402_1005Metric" (layer "F.Cu") (at 163.5 111)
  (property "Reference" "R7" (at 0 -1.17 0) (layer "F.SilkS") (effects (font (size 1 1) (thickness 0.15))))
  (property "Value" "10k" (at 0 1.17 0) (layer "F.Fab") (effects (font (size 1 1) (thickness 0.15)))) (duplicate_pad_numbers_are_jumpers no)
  (pad "1" smd roundrect (at -0.51 0) (size 0.54 0.64) (layers "F.Cu" "F.Mask" "F.Paste") (roundrect_rratio 0.25) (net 12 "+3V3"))
  (pad "2" smd roundrect (at 0.51 0) (size 0.54 0.64) (layers "F.Cu" "F.Mask" "F.Paste") (roundrect_rratio 0.25) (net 34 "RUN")))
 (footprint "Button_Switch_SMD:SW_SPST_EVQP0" (layer "F.Cu") (at 169.5 107)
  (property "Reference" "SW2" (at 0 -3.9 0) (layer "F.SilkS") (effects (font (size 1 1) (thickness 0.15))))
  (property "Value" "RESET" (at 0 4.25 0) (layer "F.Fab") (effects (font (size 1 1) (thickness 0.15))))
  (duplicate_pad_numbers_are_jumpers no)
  (pad "1" smd rect (at -2.88 -2) (size 2.75 1) (layers "F.Cu" "F.Mask" "F.Paste") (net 34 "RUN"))
  (pad "1" smd rect (at 2.88 -2) (size 2.75 1) (layers "F.Cu" "F.Mask" "F.Paste") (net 34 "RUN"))
  (pad "2" smd rect (at -2.88 2) (size 2.75 1) (layers "F.Cu" "F.Mask" "F.Paste") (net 1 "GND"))
  (pad "2" smd rect (at 2.88 2) (size 2.75 1) (layers "F.Cu" "F.Mask" "F.Paste") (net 1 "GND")))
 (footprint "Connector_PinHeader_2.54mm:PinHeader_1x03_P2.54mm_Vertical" (layer "F.Cu") (at 175 115)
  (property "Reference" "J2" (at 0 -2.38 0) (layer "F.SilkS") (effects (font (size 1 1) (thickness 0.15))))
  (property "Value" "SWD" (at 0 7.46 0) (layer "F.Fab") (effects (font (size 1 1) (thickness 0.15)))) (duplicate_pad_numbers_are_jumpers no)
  (pad "1" thru_hole rect (at 0 0) (size 1.7 1.7) (drill 1) (layers "*.Cu" "*.Mask") (remove_unused_layers no) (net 32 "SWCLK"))
  (pad "2" thru_hole circle (at 0 2.54) (size 1.7 1.7) (drill 1) (layers "*.Cu" "*.Mask") (remove_unused_layers no) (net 1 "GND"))
  (pad "3" thru_hole circle (at 0 5.08) (size 1.7 1.7) (drill 1) (layers "*.Cu" "*.Mask") (remove_unused_layers no) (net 33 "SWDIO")))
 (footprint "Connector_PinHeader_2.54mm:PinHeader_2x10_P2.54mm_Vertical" (layer "F.Cu") (at 146.5 123.5 90)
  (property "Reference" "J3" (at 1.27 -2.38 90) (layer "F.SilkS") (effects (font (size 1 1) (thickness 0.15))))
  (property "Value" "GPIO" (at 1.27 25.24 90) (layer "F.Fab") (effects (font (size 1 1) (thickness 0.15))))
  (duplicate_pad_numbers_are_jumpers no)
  (pad "1" thru_hole rect (at 0 0 90) (size 1.7 1.7) (drill 1) (layers "*.Cu" "*.Mask") (remove_unused_layers no) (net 13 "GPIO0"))
  (pad "2" thru_hole circle (at 2.54 0 90) (size 1.7 1.7) (drill 1) (layers "*.Cu" "*.Mask") (remove_unused_layers no) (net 14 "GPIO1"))
  (pad "3" thru_hole circle (at 0 2.54 90) (size 1.7 1.7) (drill 1) (layers "*.Cu" "*.Mask") (remove_unused_layers no) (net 15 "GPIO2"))
  (pad "4" thru_hole circle (at 2.54 2.54 90) (size 1.7 1.7) (drill 1) (layers "*.Cu" "*.Mask") (remove_unused_layers no) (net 16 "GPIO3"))
  (pad "5" thru_hole circle (at 0 5.08 90) (size 1.7 1.7) (drill 1) (layers "*.Cu" "*.Mask") (remove_unused_layers no) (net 17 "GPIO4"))
  (pad "6" thru_hole circle (at 2.54 5.08 90) (size 1.7 1.7) (drill 1) (layers "*.Cu" "*.Mask") (remove_unused_layers no) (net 18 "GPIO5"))
  (pad "7" thru_hole circle (at 0 7.62 90) (size 1.7 1.7) (drill 1) (layers "*.Cu" "*.Mask") (remove_unused_layers no) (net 19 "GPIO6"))
  (pad "8" thru_hole circle (at 2.54 7.62 90) (size 1.7 1.7) (drill 1) (layers "*.Cu" "*.Mask") (remove_unused_layers no) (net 20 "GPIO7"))
  (pad "9" thru_hole circle (at 0 10.16 90) (size 1.7 1.7) (drill 1) (layers "*.Cu" "*.Mask") (remove_unused_layers no) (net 21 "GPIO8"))
  (pad "10" thru_hole circle (at 2.54 10.16 90) (size 1.7 1.7) (drill 1) (layers "*.Cu" "*.Mask") (remove_unused_layers no) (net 22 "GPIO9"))
  (pad "11" thru_hole circle (at 0 12.7 90) (size 1.7 1.7) (drill 1) (layers "*.Cu" "*.Mask") (remove_unused_layers no) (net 23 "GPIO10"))
  (pad "12" thru_hole circle (at 2.54 12.7 90) (size 1.7 1.7) (drill 1) (layers "*.Cu" "*.Mask") (remove_unused_layers no) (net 24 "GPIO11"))
  (pad "13" thru_hole circle (at 0 15.24 90) (size 1.7 1.7) (drill 1) (layers "*.Cu" "*.Mask") (remove_unused_layers no) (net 25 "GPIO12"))
  (pad "14" thru_hole circle (at 2.54 15.24 90) (size 1.7 1.7) (drill 1) (layers "*.Cu" "*.Mask") (remove_unused_layers no)
   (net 26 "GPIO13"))
  (pad "15" thru_hole circle (at 0 17.78 90) (size 1.7 1.7) (drill 1) (layers "*.Cu" "*.Mask") (remove_unused_layers no) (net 27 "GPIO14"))
  (pad "16" thru_hole circle (at 2.54 17.78 90) (size 1.7 1.7) (drill 1) (layers "*.Cu" "*.Mask") (remove_unused_layers no)
   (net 28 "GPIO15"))
  (pad "17" thru_hole circle (at 0 20.32 90) (size 1.7 1.7) (drill 1) (layers "*.Cu" "*.Mask") (remove_unused_layers no) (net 45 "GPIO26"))
  (pad "18" thru_hole circle (at 2.54 20.32 90) (size 1.7 1.7) (drill 1) (layers "*.Cu" "*.Mask") (remove_unused_layers no)
   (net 46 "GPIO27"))
  (pad "19" thru_hole circle (at 0 22.86 90) (size 1.7 1.7) (drill 1) (layers "*.Cu" "*.Mask") (remove_unused_layers no) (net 47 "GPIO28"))
  (pad "20" thru_hole circle (at 2.54 22.86 90) (size 1.7 1.7) (drill 1) (layers "*.Cu" "*.Mask") (remove_unused_layers no)
   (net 48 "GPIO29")))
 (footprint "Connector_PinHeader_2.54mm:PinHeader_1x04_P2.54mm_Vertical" (layer "F.Cu") (at 122 110)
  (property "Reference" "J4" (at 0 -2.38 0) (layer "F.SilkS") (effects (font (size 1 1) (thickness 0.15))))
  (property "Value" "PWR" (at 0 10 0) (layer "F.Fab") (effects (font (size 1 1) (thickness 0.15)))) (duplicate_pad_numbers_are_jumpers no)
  (pad "1" thru_hole rect (at 0 0) (size 1.7 1.7) (drill 1) (layers "*.Cu" "*.Mask") (remove_unused_layers no) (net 2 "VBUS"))
  (pad "2" thru_hole circle (at 0 2.54) (size 1.7 1.7) (drill 1) (layers "*.Cu" "*.Mask") (remove_unused_layers no) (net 12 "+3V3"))
  (pad "3" thru_hole circle (at 0 5.08) (size 1.7 1.7) (drill 1) (layers "*.Cu" "*.Mask") (remove_unused_layers no) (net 1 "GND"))
  (pad "4" thru_hole circle (at 0 7.62) (size 1.7 1.7) (drill 1) (layers "*.Cu" "*.Mask") (remove_unused_layers no) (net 1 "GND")))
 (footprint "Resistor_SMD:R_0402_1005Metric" (layer "F.Cu") (at 128.5 106)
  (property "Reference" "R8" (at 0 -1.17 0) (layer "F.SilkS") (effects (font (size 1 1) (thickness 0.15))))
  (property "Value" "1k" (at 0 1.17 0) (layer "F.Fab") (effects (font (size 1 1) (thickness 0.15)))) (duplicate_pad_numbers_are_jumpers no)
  (pad "1" smd roundrect (at -0.51 0) (size 0.54 0.64) (layers "F.Cu" "F.Mask" "F.Paste") (roundrect_rratio 0.25) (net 12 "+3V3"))
  (pad "2" smd roundrect (at 0.51 0) (size 0.54 0.64) (layers "F.Cu" "F.Mask" "F.Paste") (roundrect_rratio 0.25) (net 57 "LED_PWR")))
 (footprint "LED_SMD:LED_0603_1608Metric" (layer "F.Cu") (at 128.5 109)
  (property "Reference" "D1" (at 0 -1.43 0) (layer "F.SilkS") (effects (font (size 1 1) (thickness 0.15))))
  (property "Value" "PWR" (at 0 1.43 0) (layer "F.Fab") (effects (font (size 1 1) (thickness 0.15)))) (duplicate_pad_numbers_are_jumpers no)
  (pad "1" smd roundrect (at -0.7875 0) (size 0.875 0.95) (layers "F.Cu" "F.Mask" "F.Paste") (roundrect_rratio 0.25) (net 1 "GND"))
  (pad "2" smd roundrect (at 0.7875 0) (size 0.875 0.95) (layers "F.Cu" "F.Mask" "F.Paste") (roundrect_rratio 0.25) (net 57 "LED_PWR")))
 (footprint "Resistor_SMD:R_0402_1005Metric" (layer "F.Cu") (at 163.5 117)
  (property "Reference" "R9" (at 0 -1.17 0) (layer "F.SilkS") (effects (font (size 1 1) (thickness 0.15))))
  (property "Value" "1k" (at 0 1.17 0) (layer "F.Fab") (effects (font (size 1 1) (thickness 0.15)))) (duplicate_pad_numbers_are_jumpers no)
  (pad "1" smd roundrect (at -0.51 0) (size 0.54 0.64) (layers "F.Cu" "F.Mask" "F.Paste") (roundrect_rratio 0.25) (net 44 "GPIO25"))
  (pad "2" smd roundrect (at 0.51 0) (size 0.54 0.64) (layers "F.Cu" "F.Mask" "F.Paste") (roundrect_rratio 0.25) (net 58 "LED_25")))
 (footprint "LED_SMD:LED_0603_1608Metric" (layer "F.Cu") (at 167.5 117)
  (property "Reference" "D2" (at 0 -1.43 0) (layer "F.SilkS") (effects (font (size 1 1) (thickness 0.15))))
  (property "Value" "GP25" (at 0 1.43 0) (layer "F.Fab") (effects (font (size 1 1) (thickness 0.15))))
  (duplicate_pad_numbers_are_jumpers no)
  (pad "1" smd roundrect (at -0.7875 0) (size 0.875 0.95) (layers "F.Cu" "F.Mask" "F.Paste") (roundrect_rratio 0.25) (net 1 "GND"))
  (pad "2" smd roundrect (at 0.7875 0) (size 0.875 0.95) (layers "F.Cu" "F.Mask" "F.Paste") (roundrect_rratio 0.25) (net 58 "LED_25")))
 (segment (start 149.1 96.11) (end 149.1 96.6) (width 0.2) (layer "F.Cu") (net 9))
 (segment (start 149.1 96.6) (end 149.5 97.0) (width 0.2) (layer "F.Cu") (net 9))
 (segment (start 149.5 97.0) (end 149.5 102.562) (width 0.2) (layer "F.Cu") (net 9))
 (segment (start 150.3 96.11) (end 150.3 96.6) (width 0.2) (layer "F.Cu") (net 10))
 (segment (start 150.3 96.6) (end 149.9 97.0) (width 0.2) (layer "F.Cu") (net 10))
 (segment (start 149.9 97.0) (end 149.9 102.562) (width 0.2) (layer "F.Cu") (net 10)))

